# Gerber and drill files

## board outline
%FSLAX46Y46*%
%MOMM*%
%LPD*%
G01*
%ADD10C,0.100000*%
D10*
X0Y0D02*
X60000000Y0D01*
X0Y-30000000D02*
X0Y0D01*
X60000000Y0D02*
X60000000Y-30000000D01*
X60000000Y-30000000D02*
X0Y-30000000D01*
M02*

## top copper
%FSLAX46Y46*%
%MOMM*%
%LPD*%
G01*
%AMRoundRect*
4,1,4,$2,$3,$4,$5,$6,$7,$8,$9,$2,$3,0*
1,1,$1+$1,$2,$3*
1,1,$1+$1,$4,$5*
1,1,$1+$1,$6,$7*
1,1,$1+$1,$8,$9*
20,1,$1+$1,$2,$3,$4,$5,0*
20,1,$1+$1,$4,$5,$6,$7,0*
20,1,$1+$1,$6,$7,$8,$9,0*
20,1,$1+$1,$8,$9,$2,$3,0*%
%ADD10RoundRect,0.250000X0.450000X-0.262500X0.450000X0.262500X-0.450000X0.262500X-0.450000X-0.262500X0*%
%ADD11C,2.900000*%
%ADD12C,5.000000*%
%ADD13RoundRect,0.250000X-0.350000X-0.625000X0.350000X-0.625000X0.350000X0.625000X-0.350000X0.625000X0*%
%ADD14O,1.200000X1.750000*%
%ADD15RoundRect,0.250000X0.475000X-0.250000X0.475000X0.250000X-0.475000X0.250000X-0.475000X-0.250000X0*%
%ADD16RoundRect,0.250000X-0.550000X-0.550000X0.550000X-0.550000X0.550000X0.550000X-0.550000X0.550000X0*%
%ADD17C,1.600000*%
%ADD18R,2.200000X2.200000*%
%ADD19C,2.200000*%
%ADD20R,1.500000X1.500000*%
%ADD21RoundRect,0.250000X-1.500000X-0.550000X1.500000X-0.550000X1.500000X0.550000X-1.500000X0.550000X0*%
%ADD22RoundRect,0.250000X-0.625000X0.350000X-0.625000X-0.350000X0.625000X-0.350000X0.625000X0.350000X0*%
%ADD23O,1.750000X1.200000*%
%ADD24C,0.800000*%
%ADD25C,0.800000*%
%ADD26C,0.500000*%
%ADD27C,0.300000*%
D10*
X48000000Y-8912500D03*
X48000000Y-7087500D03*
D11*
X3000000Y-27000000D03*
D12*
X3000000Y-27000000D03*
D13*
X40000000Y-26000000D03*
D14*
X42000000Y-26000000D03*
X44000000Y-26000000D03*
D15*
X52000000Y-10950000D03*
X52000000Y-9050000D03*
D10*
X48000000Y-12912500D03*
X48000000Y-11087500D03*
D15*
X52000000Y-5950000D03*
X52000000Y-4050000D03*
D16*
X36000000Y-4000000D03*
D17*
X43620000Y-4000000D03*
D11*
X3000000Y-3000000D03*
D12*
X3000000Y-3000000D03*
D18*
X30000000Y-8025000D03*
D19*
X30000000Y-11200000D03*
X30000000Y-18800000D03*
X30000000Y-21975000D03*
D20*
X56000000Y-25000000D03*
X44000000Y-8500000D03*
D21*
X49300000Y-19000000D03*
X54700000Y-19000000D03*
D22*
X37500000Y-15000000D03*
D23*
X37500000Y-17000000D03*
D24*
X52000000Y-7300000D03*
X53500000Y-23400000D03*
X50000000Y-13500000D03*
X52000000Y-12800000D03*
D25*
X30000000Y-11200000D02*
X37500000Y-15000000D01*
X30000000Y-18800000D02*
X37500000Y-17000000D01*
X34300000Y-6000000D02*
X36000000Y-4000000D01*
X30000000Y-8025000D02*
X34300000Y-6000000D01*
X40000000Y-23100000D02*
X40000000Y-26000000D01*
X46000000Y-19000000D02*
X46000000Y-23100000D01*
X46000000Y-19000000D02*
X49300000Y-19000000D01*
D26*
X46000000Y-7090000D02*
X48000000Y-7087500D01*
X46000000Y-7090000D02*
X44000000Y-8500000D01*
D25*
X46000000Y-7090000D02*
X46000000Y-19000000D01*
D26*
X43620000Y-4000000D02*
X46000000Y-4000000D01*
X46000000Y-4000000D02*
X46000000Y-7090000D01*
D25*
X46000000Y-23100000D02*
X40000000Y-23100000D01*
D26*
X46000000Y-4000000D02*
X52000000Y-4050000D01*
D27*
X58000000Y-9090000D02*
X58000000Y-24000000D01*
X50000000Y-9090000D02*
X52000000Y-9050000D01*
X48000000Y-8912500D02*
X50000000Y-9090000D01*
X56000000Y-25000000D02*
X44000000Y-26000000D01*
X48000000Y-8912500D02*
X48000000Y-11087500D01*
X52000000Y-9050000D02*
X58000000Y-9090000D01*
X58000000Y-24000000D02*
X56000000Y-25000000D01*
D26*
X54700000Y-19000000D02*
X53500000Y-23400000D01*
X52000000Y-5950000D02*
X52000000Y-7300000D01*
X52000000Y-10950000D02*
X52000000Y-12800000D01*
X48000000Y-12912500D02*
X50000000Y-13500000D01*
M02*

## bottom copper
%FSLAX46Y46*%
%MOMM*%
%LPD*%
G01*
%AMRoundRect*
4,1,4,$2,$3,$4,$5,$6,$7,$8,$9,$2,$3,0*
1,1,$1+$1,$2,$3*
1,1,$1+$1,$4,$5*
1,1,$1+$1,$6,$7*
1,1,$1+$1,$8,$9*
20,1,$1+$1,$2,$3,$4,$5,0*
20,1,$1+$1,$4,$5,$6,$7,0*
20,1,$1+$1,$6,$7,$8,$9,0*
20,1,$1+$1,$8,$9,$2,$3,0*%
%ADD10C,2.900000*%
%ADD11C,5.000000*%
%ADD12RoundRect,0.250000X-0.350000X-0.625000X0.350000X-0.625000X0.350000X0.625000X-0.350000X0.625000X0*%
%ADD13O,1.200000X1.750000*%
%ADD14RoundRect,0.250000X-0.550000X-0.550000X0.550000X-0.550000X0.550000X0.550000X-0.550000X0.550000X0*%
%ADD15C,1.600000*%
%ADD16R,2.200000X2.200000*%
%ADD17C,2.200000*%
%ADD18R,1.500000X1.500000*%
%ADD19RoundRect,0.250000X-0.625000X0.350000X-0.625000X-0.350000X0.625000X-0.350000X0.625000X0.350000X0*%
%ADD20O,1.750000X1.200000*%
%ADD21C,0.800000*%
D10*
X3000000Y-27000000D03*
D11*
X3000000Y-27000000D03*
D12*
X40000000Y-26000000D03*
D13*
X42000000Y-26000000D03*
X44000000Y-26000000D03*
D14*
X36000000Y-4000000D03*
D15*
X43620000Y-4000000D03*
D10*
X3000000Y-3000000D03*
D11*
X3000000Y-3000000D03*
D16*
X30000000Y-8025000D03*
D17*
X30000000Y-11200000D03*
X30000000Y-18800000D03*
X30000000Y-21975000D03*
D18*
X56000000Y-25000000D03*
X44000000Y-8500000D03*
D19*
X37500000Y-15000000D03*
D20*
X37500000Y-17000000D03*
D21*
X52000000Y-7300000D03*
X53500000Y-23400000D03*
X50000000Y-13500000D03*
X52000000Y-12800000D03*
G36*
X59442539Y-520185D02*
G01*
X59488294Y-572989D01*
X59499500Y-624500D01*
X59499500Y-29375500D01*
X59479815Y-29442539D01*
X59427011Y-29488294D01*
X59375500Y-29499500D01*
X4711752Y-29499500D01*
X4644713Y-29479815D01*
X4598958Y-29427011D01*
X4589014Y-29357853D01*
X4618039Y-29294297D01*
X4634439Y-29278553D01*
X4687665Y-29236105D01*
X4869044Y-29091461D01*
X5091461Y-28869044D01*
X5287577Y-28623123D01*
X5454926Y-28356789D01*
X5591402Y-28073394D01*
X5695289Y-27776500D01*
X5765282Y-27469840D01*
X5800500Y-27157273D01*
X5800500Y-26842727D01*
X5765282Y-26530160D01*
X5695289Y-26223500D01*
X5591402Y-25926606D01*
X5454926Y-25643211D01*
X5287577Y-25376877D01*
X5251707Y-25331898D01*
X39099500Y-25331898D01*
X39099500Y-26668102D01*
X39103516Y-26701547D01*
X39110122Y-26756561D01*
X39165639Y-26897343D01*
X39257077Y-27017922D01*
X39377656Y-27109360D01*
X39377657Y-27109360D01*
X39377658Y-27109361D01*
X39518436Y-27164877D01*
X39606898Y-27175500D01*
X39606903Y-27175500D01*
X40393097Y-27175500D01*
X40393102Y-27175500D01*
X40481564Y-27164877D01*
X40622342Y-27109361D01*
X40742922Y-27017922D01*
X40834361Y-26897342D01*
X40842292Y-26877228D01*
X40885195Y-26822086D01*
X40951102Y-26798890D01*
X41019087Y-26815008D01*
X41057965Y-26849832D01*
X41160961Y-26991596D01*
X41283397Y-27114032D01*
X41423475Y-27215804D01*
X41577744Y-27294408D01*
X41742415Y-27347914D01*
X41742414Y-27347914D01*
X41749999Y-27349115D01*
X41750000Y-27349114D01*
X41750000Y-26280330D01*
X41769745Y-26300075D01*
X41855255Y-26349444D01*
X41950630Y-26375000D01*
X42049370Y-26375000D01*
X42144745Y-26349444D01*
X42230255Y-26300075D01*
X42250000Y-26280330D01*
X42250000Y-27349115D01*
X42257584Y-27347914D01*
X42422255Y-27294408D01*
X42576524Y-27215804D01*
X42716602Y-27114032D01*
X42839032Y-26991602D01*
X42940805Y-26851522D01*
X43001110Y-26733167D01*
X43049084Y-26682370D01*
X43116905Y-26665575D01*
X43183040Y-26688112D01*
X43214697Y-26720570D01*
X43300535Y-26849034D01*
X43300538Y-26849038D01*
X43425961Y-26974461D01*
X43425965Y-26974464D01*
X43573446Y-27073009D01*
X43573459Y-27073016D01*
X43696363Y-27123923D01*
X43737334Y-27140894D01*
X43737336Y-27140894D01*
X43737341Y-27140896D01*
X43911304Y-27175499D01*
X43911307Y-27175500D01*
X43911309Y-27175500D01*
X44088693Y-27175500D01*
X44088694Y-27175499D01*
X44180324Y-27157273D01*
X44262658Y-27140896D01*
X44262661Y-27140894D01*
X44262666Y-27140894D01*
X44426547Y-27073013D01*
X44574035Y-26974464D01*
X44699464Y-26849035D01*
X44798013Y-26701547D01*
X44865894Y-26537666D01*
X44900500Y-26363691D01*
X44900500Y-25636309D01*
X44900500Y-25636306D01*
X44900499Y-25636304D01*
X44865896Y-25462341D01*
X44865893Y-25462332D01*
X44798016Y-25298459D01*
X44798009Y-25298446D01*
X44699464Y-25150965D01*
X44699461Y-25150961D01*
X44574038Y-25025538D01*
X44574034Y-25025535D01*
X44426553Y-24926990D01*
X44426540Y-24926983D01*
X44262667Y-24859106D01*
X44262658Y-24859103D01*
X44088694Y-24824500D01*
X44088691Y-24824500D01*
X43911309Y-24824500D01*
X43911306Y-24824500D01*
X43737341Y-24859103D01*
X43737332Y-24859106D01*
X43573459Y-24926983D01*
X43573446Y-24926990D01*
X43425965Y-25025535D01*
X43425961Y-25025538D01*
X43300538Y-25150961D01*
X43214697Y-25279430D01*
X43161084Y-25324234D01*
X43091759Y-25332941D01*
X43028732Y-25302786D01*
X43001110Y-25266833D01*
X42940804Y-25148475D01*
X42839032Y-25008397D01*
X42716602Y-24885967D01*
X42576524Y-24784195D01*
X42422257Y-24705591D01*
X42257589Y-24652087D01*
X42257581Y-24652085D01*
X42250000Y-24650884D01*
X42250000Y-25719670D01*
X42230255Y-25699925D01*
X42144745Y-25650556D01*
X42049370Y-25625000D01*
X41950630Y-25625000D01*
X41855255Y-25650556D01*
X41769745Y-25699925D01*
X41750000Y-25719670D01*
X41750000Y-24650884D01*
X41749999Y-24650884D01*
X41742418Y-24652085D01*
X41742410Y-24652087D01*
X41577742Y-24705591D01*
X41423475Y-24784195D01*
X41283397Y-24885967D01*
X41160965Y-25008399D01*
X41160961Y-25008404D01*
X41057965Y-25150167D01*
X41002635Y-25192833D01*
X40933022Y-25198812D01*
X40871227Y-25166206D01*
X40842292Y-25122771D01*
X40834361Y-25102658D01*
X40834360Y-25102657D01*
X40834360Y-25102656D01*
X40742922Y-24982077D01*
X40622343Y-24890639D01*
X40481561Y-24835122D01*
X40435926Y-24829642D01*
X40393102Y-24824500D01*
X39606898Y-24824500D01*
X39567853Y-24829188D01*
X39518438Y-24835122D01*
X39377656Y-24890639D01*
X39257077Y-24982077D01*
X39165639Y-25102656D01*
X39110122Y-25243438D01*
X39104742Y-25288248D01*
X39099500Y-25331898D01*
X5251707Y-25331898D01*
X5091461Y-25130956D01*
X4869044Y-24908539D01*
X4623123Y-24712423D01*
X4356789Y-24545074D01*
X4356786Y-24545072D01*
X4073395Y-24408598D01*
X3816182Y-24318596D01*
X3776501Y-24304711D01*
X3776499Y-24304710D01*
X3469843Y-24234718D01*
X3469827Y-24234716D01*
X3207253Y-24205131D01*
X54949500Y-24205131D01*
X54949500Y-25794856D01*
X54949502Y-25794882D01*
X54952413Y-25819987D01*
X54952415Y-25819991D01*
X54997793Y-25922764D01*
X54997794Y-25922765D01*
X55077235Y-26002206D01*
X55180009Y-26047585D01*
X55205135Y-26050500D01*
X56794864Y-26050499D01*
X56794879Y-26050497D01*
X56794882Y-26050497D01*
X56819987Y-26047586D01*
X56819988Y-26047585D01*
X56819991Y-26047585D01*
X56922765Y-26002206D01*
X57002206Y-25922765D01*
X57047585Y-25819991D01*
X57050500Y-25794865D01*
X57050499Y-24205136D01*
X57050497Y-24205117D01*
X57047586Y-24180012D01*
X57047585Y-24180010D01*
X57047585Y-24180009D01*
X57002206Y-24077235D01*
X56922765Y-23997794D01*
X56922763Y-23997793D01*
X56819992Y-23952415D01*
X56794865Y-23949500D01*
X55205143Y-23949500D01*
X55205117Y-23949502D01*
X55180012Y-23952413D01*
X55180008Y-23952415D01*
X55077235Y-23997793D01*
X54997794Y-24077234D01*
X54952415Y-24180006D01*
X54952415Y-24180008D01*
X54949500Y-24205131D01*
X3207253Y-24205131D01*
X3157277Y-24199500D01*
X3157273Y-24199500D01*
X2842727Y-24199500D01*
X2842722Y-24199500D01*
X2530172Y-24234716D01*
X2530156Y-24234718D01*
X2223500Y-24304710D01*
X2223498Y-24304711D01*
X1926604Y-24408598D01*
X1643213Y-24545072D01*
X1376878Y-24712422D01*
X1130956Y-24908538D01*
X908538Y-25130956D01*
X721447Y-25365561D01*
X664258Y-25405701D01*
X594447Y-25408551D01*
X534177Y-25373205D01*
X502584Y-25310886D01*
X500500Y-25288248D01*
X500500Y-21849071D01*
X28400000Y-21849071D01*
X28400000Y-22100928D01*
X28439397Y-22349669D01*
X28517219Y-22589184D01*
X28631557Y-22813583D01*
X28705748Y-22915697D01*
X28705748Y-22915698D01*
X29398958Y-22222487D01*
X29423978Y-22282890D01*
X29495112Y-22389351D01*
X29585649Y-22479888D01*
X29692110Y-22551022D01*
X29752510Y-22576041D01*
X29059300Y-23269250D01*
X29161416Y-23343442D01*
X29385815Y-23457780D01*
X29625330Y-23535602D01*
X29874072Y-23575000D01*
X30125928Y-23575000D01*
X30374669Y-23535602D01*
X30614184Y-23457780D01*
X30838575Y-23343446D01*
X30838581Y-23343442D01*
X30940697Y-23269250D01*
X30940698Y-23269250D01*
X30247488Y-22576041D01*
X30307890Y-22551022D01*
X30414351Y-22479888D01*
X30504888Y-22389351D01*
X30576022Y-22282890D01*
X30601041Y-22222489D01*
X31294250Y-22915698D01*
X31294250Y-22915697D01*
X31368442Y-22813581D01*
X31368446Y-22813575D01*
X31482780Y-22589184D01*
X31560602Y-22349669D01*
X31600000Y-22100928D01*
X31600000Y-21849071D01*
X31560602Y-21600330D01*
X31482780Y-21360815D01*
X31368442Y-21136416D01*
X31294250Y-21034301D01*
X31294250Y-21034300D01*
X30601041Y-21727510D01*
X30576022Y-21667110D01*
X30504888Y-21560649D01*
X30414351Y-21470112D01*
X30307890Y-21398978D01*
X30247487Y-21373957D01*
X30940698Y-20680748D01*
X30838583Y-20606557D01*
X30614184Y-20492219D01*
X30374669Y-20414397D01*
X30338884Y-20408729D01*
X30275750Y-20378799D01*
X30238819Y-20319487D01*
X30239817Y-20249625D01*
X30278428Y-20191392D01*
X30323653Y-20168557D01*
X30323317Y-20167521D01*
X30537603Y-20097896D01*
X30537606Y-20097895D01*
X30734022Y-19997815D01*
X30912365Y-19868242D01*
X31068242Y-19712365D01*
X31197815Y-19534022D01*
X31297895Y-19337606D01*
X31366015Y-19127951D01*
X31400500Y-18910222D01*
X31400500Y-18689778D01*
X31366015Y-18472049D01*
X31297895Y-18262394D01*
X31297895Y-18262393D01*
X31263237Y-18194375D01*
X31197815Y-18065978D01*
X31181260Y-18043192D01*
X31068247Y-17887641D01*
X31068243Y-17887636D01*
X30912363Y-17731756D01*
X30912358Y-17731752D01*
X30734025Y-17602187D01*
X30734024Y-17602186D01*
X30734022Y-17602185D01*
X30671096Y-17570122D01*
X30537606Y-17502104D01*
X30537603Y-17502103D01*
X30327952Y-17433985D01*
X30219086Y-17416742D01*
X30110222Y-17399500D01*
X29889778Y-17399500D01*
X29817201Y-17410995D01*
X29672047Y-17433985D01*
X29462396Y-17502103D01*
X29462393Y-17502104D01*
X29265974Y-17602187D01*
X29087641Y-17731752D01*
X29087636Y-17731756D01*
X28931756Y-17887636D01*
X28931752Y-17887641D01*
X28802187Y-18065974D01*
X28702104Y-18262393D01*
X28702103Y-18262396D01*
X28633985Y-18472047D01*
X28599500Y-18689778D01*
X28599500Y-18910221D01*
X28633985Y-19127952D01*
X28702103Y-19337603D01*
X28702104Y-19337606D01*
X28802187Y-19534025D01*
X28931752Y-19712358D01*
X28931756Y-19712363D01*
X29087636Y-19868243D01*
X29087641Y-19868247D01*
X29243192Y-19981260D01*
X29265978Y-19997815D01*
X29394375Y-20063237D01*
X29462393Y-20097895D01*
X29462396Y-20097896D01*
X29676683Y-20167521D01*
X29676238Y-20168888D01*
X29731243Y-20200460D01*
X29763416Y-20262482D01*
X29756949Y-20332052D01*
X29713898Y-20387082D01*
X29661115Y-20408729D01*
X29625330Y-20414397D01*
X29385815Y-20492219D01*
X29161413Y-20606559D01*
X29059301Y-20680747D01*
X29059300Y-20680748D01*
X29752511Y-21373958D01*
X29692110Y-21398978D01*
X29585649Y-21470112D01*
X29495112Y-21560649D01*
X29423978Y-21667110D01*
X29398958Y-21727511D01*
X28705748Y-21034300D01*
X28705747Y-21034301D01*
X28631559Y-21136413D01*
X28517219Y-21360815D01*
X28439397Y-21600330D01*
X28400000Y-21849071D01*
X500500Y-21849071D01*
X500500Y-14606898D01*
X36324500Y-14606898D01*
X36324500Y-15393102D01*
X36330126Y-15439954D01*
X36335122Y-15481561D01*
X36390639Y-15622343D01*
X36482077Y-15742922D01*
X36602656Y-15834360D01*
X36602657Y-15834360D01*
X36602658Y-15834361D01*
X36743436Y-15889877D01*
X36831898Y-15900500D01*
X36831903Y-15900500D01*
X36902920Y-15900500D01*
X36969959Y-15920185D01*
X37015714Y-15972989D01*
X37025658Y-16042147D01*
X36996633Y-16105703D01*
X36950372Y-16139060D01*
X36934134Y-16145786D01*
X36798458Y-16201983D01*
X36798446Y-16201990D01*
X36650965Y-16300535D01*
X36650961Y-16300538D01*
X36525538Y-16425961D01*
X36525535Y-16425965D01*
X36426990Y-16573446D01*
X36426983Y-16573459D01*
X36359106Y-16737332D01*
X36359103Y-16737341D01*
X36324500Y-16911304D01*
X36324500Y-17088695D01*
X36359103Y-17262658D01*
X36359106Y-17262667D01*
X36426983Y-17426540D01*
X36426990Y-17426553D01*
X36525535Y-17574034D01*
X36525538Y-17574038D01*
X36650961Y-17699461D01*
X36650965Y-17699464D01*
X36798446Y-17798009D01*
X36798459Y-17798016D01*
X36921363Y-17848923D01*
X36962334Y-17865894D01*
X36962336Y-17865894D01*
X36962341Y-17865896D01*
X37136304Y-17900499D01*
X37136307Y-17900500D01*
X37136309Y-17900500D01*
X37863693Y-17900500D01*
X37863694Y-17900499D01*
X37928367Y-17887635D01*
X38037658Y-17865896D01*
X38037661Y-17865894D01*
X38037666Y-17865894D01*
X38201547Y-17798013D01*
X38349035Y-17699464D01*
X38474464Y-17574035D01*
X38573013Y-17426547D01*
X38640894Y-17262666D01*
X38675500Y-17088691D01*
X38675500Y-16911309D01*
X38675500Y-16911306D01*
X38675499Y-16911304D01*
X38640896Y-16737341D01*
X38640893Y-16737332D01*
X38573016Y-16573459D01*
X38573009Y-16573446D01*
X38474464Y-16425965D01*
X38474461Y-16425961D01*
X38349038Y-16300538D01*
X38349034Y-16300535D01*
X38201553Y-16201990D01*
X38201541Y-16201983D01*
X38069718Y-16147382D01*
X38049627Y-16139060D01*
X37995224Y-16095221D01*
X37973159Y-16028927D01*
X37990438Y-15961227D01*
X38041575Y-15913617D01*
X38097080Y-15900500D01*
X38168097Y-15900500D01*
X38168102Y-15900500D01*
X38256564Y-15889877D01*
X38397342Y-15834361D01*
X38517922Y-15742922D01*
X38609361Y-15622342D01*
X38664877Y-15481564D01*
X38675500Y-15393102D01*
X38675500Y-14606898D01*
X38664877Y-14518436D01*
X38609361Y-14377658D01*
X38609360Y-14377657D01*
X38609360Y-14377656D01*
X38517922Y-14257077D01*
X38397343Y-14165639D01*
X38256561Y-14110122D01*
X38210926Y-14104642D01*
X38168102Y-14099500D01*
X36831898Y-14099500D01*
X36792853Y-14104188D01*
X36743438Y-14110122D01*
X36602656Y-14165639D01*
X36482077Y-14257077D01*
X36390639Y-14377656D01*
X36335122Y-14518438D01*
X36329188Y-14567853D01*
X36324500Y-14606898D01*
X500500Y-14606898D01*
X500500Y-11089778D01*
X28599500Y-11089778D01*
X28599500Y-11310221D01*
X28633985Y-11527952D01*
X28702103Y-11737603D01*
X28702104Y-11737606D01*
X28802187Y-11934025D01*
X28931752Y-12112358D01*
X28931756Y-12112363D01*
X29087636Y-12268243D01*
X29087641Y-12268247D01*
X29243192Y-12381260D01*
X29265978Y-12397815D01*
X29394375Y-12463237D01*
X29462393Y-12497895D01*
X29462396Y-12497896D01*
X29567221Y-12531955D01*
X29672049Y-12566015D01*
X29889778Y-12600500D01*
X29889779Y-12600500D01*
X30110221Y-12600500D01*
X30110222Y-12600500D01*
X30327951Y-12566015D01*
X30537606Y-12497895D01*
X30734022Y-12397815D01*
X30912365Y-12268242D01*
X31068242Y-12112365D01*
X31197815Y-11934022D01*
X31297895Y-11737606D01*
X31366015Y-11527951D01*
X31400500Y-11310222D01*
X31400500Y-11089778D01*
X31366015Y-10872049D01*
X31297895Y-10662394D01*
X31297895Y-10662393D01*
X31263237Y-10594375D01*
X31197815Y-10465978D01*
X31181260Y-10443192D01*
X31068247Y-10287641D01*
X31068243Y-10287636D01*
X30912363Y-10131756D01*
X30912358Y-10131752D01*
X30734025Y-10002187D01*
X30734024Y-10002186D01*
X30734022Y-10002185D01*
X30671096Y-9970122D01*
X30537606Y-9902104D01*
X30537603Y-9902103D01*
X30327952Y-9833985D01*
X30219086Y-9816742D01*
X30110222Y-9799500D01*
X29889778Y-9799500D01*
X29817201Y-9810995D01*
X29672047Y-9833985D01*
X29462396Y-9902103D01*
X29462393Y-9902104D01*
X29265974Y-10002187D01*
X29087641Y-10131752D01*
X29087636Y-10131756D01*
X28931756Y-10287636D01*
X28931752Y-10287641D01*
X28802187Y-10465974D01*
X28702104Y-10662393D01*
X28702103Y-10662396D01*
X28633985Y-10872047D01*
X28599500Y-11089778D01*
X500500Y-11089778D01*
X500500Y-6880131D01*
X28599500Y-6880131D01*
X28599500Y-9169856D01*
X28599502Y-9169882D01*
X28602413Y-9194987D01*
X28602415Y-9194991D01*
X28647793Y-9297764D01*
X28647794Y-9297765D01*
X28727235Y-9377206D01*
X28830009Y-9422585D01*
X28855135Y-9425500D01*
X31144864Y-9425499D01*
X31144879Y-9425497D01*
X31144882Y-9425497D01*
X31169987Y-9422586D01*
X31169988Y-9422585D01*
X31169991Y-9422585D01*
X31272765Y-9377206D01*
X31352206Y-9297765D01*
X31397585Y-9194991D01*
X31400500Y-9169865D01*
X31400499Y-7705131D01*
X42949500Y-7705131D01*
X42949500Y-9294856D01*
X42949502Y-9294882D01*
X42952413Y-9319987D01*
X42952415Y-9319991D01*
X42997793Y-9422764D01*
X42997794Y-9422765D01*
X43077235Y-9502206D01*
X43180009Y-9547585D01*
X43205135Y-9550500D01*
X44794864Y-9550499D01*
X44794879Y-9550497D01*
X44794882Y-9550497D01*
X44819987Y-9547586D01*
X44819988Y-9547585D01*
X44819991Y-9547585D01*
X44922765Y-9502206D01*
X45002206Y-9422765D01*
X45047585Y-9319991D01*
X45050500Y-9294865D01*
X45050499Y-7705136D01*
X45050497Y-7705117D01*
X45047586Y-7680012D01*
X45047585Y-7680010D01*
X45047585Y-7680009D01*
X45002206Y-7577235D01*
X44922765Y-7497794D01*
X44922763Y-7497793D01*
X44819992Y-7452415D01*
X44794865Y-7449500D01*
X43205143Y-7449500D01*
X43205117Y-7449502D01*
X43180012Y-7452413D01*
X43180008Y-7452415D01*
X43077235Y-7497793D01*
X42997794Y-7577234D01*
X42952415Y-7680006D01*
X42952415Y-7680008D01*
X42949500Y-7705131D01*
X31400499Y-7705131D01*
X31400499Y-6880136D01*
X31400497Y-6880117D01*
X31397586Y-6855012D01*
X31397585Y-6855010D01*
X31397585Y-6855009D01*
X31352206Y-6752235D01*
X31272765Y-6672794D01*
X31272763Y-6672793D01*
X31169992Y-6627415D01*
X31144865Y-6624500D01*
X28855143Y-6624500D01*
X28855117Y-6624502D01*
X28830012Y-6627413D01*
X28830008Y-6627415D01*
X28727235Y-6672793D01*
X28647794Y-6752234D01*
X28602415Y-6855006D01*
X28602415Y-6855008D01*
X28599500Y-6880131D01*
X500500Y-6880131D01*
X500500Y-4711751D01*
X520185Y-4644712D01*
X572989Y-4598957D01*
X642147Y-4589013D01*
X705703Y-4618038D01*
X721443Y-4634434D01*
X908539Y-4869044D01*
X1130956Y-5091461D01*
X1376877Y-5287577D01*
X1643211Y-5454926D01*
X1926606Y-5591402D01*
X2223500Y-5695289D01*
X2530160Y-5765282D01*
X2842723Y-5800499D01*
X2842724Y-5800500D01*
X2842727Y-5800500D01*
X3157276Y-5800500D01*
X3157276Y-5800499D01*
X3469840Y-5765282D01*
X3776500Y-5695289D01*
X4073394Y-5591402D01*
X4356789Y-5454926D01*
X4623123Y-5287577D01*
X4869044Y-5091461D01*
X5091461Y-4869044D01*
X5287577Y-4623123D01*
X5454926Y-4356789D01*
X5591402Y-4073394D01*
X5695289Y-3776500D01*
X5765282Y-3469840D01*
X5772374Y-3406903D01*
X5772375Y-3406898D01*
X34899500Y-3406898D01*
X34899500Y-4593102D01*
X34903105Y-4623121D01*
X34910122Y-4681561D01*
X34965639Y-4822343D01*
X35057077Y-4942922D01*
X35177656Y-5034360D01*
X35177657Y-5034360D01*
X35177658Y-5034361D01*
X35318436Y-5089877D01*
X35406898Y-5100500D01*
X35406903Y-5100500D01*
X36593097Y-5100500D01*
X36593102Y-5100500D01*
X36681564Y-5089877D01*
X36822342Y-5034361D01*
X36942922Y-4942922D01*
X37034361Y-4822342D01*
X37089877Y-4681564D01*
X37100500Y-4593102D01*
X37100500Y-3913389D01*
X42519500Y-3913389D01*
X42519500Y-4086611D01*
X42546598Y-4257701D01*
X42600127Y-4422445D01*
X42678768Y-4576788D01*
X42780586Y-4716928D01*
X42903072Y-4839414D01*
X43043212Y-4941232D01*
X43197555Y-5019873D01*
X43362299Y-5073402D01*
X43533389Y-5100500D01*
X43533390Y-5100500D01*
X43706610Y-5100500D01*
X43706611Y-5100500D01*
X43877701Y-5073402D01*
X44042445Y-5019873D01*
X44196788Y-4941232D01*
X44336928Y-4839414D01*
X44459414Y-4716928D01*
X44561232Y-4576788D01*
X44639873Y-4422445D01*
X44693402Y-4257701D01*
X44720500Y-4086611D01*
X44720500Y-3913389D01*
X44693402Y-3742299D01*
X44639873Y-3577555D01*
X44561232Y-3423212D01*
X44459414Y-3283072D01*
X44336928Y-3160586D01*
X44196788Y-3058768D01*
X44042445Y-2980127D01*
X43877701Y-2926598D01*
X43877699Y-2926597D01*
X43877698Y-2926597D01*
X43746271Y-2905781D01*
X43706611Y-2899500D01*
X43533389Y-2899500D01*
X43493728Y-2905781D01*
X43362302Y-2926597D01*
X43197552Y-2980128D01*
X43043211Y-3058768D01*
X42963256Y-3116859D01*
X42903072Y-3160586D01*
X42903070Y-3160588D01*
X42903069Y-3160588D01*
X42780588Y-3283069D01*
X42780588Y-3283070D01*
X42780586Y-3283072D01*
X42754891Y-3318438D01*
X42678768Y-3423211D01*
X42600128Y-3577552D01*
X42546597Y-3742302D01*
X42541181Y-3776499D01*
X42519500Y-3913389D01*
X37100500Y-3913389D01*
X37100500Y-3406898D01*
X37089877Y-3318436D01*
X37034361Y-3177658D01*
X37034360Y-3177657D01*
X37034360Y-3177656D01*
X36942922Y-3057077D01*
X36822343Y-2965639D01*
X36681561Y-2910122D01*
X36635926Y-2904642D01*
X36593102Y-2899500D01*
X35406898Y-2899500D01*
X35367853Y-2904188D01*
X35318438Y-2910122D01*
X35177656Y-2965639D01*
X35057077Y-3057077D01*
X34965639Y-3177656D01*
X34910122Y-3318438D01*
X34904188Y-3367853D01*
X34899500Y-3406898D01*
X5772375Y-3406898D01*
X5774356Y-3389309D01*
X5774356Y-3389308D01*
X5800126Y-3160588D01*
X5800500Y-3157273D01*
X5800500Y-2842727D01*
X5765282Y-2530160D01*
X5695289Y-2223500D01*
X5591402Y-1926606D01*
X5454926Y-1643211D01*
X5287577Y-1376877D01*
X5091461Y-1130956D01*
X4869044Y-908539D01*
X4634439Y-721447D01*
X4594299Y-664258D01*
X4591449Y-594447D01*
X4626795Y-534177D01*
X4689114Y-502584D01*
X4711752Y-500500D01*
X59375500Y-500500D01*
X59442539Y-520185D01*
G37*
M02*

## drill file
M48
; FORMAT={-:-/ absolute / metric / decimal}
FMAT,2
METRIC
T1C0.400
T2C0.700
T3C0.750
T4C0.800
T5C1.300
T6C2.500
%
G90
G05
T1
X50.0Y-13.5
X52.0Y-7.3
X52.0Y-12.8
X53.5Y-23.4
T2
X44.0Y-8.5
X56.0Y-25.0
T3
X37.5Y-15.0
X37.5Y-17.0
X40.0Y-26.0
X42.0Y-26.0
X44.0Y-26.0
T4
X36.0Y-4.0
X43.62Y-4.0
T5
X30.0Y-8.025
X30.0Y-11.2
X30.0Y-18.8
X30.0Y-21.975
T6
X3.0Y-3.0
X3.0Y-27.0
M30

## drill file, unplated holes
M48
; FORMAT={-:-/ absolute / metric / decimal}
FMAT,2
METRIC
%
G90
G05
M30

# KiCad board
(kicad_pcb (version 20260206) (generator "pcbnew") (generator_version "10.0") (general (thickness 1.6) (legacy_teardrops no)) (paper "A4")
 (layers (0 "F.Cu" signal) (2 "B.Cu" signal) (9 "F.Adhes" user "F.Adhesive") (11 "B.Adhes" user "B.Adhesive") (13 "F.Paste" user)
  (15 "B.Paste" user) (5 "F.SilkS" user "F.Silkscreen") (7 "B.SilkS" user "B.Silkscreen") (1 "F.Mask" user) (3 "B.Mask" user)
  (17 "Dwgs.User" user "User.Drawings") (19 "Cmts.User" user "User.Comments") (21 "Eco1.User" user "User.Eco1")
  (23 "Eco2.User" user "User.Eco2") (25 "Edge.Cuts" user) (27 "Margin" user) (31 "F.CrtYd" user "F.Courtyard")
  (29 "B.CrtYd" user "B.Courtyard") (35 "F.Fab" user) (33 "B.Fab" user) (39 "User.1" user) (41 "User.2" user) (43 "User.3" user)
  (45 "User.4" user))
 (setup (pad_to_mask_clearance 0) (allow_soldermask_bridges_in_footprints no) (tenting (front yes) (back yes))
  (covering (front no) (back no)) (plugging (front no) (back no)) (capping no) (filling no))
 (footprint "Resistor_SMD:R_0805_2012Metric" (layer "F.Cu") (at 48 8 90)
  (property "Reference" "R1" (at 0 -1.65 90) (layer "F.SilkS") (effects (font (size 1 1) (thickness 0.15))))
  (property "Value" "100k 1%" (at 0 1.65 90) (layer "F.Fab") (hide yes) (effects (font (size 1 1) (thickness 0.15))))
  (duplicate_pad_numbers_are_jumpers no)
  (pad "1" smd roundrect (at -0.9125 0 90) (size 1.025 1.4) (layers "F.Cu" "F.Mask" "F.Paste") (roundrect_rratio 0.243902) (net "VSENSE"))
  (pad "2" smd roundrect (at 0.9125 0 90) (size 1.025 1.4) (layers "F.Cu" "F.Mask" "F.Paste") (roundrect_rratio 0.243902) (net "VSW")))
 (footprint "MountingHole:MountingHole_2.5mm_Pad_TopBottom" (layer "F.Cu") (at 3 27)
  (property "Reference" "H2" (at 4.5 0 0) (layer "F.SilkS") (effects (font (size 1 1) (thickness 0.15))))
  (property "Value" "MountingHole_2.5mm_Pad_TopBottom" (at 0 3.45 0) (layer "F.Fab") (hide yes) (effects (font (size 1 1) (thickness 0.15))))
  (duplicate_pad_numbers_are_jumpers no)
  (pad "1" thru_hole circle (at 0 0) (size 2.9 2.9) (drill 2.5) (layers "*.Cu" "*.Mask") (remove_unused_layers no) (zone_connect 2))
  (pad "1" connect circle (at 0 0) (size 5 5) (layers "F.Cu" "F.Mask") (zone_connect 2))
  (pad "1" connect circle (at 0 0) (size 5 5) (layers "B.Cu" "B.Mask") (zone_connect 2)))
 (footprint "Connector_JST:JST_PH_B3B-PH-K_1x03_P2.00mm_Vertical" (layer "F.Cu") (at 40 26)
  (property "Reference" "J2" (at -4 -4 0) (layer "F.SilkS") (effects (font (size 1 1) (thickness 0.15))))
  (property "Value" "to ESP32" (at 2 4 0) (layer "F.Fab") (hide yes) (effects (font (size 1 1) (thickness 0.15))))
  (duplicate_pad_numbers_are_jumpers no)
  (pad "1" thru_hole roundrect (at 0 0) (size 1.2 1.75) (drill 0.75) (layers "*.Cu" "*.Mask") (remove_unused_layers no)
   (roundrect_rratio 0.208333) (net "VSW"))
  (pad "2" thru_hole oval (at 2 0) (size 1.2 1.75) (drill 0.75) (layers "*.Cu" "*.Mask") (remove_unused_layers no) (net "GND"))
  (pad "3" thru_hole oval (at 4 0) (size 1.2 1.75) (drill 0.75) (layers "*.Cu" "*.Mask") (remove_unused_layers no) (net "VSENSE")))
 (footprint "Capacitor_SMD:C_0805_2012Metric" (layer "F.Cu") (at 52 10 90)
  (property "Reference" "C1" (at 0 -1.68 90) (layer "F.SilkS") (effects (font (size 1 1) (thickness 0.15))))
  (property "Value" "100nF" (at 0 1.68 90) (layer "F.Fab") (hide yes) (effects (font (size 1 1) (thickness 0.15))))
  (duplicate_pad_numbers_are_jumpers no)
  (pad "1" smd roundrect (at -0.95 0 90) (size 1 1.45) (layers "F.Cu" "F.Mask" "F.Paste") (roundrect_rratio 0.25) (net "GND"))
  (pad "2" smd roundrect (at 0.95 0 90) (size 1 1.45) (layers "F.Cu" "F.Mask" "F.Paste") (roundrect_rratio 0.25) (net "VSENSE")))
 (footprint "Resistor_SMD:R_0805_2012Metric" (layer "F.Cu") (at 48 12 90)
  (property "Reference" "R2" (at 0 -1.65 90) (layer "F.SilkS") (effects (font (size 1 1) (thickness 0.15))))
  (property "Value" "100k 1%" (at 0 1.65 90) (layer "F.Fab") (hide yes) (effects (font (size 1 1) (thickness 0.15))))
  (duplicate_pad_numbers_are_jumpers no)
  (pad "1" smd roundrect (at -0.9125 0 90) (size 1.025 1.4) (layers "F.Cu" "F.Mask" "F.Paste") (roundrect_rratio 0.243902) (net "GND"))
  (pad "2" smd roundrect (at 0.9125 0 90) (size 1.025 1.4) (layers "F.Cu" "F.Mask" "F.Paste") (roundrect_rratio 0.243902) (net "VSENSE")))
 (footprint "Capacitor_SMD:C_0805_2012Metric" (layer "F.Cu") (at 52 5 90)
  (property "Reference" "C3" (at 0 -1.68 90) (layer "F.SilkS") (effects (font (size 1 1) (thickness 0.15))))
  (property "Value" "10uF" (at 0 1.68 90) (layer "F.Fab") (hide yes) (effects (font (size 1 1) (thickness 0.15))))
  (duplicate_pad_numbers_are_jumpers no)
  (pad "1" smd roundrect (at -0.95 0 90) (size 1 1.45) (layers "F.Cu" "F.Mask" "F.Paste") (roundrect_rratio 0.25) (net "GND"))
  (pad "2" smd roundrect (at 0.95 0 90) (size 1 1.45) (layers "F.Cu" "F.Mask" "F.Paste") (roundrect_rratio 0.25) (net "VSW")))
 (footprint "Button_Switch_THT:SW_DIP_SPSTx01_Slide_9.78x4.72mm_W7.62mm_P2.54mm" (layer "F.Cu") (at 36 4)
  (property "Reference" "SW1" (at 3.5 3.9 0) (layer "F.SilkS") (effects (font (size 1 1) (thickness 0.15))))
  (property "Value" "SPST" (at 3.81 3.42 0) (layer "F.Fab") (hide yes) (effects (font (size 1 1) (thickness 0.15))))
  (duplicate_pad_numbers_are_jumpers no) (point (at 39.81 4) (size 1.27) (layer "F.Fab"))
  (pad "1" thru_hole roundrect (at 0 0) (size 1.6 1.6) (drill 0.8) (layers "*.Cu" "*.Mask") (remove_unused_layers no)
   (roundrect_rratio 0.15625) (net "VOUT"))
  (pad "2" thru_hole circle (at 7.62 0) (size 1.6 1.6) (drill 0.8) (layers "*.Cu" "*.Mask") (remove_unused_layers no) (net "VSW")))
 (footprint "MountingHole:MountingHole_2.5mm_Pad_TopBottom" (layer "F.Cu") (at 3 3)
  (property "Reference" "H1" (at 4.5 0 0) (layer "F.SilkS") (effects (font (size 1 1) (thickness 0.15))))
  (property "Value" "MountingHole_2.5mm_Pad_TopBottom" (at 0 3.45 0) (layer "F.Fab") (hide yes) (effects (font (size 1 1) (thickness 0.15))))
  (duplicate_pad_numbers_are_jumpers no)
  (pad "1" thru_hole circle (at 0 0) (size 2.9 2.9) (drill 2.5) (layers "*.Cu" "*.Mask") (remove_unused_layers no) (zone_connect 2))
  (pad "1" connect circle (at 0 0) (size 5 5) (layers "F.Cu" "F.Mask") (zone_connect 2))
  (pad "1" connect circle (at 0 0) (size 5 5) (layers "B.Cu" "B.Mask") (zone_connect 2)))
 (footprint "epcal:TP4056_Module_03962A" (layer "F.Cu") (at 30 15)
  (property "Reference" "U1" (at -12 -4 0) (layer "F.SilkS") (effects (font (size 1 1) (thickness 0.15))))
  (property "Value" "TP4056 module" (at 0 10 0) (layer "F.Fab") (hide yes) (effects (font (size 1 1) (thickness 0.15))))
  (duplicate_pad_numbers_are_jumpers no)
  (pad "1" thru_hole rect (at 0 -6.975) (size 2.2 2.2) (drill 1.3) (layers "*.Cu" "*.Mask") (remove_unused_layers no) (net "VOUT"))
  (pad "2" thru_hole circle (at 0 -3.8) (size 2.2 2.2) (drill 1.3) (layers "*.Cu" "*.Mask") (remove_unused_layers no) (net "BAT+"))
  (pad "3" thru_hole circle (at 0 3.8) (size 2.2 2.2) (drill 1.3) (layers "*.Cu" "*.Mask") (remove_unused_layers no) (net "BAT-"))
  (pad "4" thru_hole circle (at 0 6.975) (size 2.2 2.2) (drill 1.3) (layers "*.Cu" "*.Mask") (remove_unused_layers no) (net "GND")))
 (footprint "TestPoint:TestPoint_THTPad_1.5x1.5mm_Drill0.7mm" (layer "F.Cu") (at 56 25)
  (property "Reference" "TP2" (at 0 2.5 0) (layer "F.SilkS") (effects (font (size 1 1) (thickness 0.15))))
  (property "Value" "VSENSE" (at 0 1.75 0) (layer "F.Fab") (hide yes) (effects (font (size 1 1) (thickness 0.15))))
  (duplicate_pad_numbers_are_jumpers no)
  (pad "1" thru_hole rect (at 0 0) (size 1.5 1.5) (drill 0.7) (layers "*.Cu" "*.Mask") (remove_unused_layers no) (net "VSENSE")))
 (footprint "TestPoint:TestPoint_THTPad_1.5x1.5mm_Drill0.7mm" (layer "F.Cu") (at 44 8.5)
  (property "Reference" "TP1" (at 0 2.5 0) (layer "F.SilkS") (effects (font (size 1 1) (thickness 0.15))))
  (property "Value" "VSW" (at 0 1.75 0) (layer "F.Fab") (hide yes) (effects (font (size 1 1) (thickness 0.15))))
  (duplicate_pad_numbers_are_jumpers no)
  (pad "1" thru_hole rect (at 0 0) (size 1.5 1.5) (drill 0.7) (layers "*.Cu" "*.Mask") (remove_unused_layers no) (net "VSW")))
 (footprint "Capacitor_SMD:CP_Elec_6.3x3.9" (layer "F.Cu") (at 52 19)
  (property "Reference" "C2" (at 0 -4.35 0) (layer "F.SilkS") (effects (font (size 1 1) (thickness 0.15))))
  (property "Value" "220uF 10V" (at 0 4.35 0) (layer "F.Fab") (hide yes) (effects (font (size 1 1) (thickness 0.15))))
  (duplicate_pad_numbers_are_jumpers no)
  (pad "1" smd roundrect (at -2.7 0) (size 3.5 1.6) (layers "F.Cu" "F.Mask" "F.Paste") (roundrect_rratio 0.15625) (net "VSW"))
  (pad "2" smd roundrect (at 2.7 0) (size 3.5 1.6) (layers "F.Cu" "F.Mask" "F.Paste") (roundrect_rratio 0.15625) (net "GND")))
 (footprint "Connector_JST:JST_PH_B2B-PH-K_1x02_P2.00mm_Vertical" (layer "F.Cu") (at 37.5 15 -90)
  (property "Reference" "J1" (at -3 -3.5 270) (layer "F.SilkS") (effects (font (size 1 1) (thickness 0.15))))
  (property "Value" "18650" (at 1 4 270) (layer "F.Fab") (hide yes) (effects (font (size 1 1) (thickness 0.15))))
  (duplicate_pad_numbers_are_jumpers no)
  (pad "1" thru_hole roundrect (at 0 0 270) (size 1.2 1.75) (drill 0.75) (layers "*.Cu" "*.Mask") (remove_unused_layers no)
   (roundrect_rratio 0.208333) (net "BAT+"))
  (pad "2" thru_hole oval (at 2 0 270) (size 1.2 1.75) (drill 0.75) (layers "*.Cu" "*.Mask") (remove_unused_layers no) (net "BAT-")))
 (gr_line (start 0 0) (end 60 0) (stroke (width 0.1) (type default)) (layer "Edge.Cuts"))
 (gr_line (start 0 30) (end 0 0) (stroke (width 0.1) (type default)) (layer "Edge.Cuts"))
 (gr_line (start 60 0) (end 60 30) (stroke (width 0.1) (type default)) (layer "Edge.Cuts"))
 (gr_line (start 60 30) (end 0 30) (stroke (width 0.1) (type default)) (layer "Edge.Cuts"))
 (segment (start 30 11.2) (end 37.5 15) (width 0.8) (layer "F.Cu") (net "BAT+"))
 (segment (start 30 18.8) (end 37.5 17) (width 0.8) (layer "F.Cu") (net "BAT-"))
 (segment (start 34.3 6) (end 36 4) (width 0.8) (layer "F.Cu") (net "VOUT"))
 (segment (start 30 8.025) (end 34.3 6) (width 0.8) (layer "F.Cu") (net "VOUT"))
 (segment (start 40 23.1) (end 40 26) (width 0.8) (layer "F.Cu") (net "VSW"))
 (segment (start 46 19) (end 46 23.1) (width 0.8) (layer "F.Cu") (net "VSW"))
 (segment (start 46 19) (end 49.3 19) (width 0.8) (layer "F.Cu") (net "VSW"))
 (segment (start 46 7.09) (end 48 7.0875) (width 0.5) (layer "F.Cu") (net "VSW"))
 (segment (start 46 7.09) (end 44 8.5) (width 0.5) (layer "F.Cu") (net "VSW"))
 (segment (start 46 7.09) (end 46 19) (width 0.8) (layer "F.Cu") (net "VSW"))
 (segment (start 43.62 4) (end 46 4) (width 0.5) (layer "F.Cu") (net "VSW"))
 (segment (start 46 4) (end 46 7.09) (width 0.5) (layer "F.Cu") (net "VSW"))
 (segment (start 46 23.1) (end 40 23.1) (width 0.8) (layer "F.Cu") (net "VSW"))
 (segment (start 46 4) (end 52 4.05) (width 0.5) (layer "F.Cu") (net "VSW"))
 (segment (start 58 9.09) (end 58 24) (width 0.3) (layer "F.Cu") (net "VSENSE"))
 (segment (start 50 9.09) (end 52 9.05) (width 0.3) (layer "F.Cu") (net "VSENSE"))
 (segment (start 48 8.9125) (end 50 9.09) (width 0.3) (layer "F.Cu") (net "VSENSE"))
 (segment (start 56 25) (end 44 26) (width 0.3) (layer "F.Cu") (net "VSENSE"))
 (segment (start 48 8.9125) (end 48 11.0875) (width 0.3) (layer "F.Cu") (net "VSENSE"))
 (segment (start 52 9.05) (end 58 9.09) (width 0.3) (layer "F.Cu") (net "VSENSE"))
 (segment (start 58 24) (end 56 25) (width 0.3) (layer "F.Cu") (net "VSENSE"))
 (segment (start 54.7 19) (end 53.5 23.4) (width 0.5) (layer "F.Cu") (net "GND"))
 (segment (start 52 5.95) (end 52 7.3) (width 0.5) (layer "F.Cu") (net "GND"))
 (segment (start 52 10.95) (end 52 12.8) (width 0.5) (layer "F.Cu") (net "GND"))
 (segment (start 48 12.9125) (end 50 13.5) (width 0.5) (layer "F.Cu") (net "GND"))
 (via (at 52 7.3) (size 0.8) (drill 0.4) (layers "F.Cu" "B.Cu") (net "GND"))
 (via (at 53.5 23.4) (size 0.8) (drill 0.4) (layers "F.Cu" "B.Cu") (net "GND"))
 (via (at 50 13.5) (size 0.8) (drill 0.4) (layers "F.Cu" "B.Cu") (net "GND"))
 (via (at 52 12.8) (size 0.8) (drill 0.4) (layers "F.Cu" "B.Cu") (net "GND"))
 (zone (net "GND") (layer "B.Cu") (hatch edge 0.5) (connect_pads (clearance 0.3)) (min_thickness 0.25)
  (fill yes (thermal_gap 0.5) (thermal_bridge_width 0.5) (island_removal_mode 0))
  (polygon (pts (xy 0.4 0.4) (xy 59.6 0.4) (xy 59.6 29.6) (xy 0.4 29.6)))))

